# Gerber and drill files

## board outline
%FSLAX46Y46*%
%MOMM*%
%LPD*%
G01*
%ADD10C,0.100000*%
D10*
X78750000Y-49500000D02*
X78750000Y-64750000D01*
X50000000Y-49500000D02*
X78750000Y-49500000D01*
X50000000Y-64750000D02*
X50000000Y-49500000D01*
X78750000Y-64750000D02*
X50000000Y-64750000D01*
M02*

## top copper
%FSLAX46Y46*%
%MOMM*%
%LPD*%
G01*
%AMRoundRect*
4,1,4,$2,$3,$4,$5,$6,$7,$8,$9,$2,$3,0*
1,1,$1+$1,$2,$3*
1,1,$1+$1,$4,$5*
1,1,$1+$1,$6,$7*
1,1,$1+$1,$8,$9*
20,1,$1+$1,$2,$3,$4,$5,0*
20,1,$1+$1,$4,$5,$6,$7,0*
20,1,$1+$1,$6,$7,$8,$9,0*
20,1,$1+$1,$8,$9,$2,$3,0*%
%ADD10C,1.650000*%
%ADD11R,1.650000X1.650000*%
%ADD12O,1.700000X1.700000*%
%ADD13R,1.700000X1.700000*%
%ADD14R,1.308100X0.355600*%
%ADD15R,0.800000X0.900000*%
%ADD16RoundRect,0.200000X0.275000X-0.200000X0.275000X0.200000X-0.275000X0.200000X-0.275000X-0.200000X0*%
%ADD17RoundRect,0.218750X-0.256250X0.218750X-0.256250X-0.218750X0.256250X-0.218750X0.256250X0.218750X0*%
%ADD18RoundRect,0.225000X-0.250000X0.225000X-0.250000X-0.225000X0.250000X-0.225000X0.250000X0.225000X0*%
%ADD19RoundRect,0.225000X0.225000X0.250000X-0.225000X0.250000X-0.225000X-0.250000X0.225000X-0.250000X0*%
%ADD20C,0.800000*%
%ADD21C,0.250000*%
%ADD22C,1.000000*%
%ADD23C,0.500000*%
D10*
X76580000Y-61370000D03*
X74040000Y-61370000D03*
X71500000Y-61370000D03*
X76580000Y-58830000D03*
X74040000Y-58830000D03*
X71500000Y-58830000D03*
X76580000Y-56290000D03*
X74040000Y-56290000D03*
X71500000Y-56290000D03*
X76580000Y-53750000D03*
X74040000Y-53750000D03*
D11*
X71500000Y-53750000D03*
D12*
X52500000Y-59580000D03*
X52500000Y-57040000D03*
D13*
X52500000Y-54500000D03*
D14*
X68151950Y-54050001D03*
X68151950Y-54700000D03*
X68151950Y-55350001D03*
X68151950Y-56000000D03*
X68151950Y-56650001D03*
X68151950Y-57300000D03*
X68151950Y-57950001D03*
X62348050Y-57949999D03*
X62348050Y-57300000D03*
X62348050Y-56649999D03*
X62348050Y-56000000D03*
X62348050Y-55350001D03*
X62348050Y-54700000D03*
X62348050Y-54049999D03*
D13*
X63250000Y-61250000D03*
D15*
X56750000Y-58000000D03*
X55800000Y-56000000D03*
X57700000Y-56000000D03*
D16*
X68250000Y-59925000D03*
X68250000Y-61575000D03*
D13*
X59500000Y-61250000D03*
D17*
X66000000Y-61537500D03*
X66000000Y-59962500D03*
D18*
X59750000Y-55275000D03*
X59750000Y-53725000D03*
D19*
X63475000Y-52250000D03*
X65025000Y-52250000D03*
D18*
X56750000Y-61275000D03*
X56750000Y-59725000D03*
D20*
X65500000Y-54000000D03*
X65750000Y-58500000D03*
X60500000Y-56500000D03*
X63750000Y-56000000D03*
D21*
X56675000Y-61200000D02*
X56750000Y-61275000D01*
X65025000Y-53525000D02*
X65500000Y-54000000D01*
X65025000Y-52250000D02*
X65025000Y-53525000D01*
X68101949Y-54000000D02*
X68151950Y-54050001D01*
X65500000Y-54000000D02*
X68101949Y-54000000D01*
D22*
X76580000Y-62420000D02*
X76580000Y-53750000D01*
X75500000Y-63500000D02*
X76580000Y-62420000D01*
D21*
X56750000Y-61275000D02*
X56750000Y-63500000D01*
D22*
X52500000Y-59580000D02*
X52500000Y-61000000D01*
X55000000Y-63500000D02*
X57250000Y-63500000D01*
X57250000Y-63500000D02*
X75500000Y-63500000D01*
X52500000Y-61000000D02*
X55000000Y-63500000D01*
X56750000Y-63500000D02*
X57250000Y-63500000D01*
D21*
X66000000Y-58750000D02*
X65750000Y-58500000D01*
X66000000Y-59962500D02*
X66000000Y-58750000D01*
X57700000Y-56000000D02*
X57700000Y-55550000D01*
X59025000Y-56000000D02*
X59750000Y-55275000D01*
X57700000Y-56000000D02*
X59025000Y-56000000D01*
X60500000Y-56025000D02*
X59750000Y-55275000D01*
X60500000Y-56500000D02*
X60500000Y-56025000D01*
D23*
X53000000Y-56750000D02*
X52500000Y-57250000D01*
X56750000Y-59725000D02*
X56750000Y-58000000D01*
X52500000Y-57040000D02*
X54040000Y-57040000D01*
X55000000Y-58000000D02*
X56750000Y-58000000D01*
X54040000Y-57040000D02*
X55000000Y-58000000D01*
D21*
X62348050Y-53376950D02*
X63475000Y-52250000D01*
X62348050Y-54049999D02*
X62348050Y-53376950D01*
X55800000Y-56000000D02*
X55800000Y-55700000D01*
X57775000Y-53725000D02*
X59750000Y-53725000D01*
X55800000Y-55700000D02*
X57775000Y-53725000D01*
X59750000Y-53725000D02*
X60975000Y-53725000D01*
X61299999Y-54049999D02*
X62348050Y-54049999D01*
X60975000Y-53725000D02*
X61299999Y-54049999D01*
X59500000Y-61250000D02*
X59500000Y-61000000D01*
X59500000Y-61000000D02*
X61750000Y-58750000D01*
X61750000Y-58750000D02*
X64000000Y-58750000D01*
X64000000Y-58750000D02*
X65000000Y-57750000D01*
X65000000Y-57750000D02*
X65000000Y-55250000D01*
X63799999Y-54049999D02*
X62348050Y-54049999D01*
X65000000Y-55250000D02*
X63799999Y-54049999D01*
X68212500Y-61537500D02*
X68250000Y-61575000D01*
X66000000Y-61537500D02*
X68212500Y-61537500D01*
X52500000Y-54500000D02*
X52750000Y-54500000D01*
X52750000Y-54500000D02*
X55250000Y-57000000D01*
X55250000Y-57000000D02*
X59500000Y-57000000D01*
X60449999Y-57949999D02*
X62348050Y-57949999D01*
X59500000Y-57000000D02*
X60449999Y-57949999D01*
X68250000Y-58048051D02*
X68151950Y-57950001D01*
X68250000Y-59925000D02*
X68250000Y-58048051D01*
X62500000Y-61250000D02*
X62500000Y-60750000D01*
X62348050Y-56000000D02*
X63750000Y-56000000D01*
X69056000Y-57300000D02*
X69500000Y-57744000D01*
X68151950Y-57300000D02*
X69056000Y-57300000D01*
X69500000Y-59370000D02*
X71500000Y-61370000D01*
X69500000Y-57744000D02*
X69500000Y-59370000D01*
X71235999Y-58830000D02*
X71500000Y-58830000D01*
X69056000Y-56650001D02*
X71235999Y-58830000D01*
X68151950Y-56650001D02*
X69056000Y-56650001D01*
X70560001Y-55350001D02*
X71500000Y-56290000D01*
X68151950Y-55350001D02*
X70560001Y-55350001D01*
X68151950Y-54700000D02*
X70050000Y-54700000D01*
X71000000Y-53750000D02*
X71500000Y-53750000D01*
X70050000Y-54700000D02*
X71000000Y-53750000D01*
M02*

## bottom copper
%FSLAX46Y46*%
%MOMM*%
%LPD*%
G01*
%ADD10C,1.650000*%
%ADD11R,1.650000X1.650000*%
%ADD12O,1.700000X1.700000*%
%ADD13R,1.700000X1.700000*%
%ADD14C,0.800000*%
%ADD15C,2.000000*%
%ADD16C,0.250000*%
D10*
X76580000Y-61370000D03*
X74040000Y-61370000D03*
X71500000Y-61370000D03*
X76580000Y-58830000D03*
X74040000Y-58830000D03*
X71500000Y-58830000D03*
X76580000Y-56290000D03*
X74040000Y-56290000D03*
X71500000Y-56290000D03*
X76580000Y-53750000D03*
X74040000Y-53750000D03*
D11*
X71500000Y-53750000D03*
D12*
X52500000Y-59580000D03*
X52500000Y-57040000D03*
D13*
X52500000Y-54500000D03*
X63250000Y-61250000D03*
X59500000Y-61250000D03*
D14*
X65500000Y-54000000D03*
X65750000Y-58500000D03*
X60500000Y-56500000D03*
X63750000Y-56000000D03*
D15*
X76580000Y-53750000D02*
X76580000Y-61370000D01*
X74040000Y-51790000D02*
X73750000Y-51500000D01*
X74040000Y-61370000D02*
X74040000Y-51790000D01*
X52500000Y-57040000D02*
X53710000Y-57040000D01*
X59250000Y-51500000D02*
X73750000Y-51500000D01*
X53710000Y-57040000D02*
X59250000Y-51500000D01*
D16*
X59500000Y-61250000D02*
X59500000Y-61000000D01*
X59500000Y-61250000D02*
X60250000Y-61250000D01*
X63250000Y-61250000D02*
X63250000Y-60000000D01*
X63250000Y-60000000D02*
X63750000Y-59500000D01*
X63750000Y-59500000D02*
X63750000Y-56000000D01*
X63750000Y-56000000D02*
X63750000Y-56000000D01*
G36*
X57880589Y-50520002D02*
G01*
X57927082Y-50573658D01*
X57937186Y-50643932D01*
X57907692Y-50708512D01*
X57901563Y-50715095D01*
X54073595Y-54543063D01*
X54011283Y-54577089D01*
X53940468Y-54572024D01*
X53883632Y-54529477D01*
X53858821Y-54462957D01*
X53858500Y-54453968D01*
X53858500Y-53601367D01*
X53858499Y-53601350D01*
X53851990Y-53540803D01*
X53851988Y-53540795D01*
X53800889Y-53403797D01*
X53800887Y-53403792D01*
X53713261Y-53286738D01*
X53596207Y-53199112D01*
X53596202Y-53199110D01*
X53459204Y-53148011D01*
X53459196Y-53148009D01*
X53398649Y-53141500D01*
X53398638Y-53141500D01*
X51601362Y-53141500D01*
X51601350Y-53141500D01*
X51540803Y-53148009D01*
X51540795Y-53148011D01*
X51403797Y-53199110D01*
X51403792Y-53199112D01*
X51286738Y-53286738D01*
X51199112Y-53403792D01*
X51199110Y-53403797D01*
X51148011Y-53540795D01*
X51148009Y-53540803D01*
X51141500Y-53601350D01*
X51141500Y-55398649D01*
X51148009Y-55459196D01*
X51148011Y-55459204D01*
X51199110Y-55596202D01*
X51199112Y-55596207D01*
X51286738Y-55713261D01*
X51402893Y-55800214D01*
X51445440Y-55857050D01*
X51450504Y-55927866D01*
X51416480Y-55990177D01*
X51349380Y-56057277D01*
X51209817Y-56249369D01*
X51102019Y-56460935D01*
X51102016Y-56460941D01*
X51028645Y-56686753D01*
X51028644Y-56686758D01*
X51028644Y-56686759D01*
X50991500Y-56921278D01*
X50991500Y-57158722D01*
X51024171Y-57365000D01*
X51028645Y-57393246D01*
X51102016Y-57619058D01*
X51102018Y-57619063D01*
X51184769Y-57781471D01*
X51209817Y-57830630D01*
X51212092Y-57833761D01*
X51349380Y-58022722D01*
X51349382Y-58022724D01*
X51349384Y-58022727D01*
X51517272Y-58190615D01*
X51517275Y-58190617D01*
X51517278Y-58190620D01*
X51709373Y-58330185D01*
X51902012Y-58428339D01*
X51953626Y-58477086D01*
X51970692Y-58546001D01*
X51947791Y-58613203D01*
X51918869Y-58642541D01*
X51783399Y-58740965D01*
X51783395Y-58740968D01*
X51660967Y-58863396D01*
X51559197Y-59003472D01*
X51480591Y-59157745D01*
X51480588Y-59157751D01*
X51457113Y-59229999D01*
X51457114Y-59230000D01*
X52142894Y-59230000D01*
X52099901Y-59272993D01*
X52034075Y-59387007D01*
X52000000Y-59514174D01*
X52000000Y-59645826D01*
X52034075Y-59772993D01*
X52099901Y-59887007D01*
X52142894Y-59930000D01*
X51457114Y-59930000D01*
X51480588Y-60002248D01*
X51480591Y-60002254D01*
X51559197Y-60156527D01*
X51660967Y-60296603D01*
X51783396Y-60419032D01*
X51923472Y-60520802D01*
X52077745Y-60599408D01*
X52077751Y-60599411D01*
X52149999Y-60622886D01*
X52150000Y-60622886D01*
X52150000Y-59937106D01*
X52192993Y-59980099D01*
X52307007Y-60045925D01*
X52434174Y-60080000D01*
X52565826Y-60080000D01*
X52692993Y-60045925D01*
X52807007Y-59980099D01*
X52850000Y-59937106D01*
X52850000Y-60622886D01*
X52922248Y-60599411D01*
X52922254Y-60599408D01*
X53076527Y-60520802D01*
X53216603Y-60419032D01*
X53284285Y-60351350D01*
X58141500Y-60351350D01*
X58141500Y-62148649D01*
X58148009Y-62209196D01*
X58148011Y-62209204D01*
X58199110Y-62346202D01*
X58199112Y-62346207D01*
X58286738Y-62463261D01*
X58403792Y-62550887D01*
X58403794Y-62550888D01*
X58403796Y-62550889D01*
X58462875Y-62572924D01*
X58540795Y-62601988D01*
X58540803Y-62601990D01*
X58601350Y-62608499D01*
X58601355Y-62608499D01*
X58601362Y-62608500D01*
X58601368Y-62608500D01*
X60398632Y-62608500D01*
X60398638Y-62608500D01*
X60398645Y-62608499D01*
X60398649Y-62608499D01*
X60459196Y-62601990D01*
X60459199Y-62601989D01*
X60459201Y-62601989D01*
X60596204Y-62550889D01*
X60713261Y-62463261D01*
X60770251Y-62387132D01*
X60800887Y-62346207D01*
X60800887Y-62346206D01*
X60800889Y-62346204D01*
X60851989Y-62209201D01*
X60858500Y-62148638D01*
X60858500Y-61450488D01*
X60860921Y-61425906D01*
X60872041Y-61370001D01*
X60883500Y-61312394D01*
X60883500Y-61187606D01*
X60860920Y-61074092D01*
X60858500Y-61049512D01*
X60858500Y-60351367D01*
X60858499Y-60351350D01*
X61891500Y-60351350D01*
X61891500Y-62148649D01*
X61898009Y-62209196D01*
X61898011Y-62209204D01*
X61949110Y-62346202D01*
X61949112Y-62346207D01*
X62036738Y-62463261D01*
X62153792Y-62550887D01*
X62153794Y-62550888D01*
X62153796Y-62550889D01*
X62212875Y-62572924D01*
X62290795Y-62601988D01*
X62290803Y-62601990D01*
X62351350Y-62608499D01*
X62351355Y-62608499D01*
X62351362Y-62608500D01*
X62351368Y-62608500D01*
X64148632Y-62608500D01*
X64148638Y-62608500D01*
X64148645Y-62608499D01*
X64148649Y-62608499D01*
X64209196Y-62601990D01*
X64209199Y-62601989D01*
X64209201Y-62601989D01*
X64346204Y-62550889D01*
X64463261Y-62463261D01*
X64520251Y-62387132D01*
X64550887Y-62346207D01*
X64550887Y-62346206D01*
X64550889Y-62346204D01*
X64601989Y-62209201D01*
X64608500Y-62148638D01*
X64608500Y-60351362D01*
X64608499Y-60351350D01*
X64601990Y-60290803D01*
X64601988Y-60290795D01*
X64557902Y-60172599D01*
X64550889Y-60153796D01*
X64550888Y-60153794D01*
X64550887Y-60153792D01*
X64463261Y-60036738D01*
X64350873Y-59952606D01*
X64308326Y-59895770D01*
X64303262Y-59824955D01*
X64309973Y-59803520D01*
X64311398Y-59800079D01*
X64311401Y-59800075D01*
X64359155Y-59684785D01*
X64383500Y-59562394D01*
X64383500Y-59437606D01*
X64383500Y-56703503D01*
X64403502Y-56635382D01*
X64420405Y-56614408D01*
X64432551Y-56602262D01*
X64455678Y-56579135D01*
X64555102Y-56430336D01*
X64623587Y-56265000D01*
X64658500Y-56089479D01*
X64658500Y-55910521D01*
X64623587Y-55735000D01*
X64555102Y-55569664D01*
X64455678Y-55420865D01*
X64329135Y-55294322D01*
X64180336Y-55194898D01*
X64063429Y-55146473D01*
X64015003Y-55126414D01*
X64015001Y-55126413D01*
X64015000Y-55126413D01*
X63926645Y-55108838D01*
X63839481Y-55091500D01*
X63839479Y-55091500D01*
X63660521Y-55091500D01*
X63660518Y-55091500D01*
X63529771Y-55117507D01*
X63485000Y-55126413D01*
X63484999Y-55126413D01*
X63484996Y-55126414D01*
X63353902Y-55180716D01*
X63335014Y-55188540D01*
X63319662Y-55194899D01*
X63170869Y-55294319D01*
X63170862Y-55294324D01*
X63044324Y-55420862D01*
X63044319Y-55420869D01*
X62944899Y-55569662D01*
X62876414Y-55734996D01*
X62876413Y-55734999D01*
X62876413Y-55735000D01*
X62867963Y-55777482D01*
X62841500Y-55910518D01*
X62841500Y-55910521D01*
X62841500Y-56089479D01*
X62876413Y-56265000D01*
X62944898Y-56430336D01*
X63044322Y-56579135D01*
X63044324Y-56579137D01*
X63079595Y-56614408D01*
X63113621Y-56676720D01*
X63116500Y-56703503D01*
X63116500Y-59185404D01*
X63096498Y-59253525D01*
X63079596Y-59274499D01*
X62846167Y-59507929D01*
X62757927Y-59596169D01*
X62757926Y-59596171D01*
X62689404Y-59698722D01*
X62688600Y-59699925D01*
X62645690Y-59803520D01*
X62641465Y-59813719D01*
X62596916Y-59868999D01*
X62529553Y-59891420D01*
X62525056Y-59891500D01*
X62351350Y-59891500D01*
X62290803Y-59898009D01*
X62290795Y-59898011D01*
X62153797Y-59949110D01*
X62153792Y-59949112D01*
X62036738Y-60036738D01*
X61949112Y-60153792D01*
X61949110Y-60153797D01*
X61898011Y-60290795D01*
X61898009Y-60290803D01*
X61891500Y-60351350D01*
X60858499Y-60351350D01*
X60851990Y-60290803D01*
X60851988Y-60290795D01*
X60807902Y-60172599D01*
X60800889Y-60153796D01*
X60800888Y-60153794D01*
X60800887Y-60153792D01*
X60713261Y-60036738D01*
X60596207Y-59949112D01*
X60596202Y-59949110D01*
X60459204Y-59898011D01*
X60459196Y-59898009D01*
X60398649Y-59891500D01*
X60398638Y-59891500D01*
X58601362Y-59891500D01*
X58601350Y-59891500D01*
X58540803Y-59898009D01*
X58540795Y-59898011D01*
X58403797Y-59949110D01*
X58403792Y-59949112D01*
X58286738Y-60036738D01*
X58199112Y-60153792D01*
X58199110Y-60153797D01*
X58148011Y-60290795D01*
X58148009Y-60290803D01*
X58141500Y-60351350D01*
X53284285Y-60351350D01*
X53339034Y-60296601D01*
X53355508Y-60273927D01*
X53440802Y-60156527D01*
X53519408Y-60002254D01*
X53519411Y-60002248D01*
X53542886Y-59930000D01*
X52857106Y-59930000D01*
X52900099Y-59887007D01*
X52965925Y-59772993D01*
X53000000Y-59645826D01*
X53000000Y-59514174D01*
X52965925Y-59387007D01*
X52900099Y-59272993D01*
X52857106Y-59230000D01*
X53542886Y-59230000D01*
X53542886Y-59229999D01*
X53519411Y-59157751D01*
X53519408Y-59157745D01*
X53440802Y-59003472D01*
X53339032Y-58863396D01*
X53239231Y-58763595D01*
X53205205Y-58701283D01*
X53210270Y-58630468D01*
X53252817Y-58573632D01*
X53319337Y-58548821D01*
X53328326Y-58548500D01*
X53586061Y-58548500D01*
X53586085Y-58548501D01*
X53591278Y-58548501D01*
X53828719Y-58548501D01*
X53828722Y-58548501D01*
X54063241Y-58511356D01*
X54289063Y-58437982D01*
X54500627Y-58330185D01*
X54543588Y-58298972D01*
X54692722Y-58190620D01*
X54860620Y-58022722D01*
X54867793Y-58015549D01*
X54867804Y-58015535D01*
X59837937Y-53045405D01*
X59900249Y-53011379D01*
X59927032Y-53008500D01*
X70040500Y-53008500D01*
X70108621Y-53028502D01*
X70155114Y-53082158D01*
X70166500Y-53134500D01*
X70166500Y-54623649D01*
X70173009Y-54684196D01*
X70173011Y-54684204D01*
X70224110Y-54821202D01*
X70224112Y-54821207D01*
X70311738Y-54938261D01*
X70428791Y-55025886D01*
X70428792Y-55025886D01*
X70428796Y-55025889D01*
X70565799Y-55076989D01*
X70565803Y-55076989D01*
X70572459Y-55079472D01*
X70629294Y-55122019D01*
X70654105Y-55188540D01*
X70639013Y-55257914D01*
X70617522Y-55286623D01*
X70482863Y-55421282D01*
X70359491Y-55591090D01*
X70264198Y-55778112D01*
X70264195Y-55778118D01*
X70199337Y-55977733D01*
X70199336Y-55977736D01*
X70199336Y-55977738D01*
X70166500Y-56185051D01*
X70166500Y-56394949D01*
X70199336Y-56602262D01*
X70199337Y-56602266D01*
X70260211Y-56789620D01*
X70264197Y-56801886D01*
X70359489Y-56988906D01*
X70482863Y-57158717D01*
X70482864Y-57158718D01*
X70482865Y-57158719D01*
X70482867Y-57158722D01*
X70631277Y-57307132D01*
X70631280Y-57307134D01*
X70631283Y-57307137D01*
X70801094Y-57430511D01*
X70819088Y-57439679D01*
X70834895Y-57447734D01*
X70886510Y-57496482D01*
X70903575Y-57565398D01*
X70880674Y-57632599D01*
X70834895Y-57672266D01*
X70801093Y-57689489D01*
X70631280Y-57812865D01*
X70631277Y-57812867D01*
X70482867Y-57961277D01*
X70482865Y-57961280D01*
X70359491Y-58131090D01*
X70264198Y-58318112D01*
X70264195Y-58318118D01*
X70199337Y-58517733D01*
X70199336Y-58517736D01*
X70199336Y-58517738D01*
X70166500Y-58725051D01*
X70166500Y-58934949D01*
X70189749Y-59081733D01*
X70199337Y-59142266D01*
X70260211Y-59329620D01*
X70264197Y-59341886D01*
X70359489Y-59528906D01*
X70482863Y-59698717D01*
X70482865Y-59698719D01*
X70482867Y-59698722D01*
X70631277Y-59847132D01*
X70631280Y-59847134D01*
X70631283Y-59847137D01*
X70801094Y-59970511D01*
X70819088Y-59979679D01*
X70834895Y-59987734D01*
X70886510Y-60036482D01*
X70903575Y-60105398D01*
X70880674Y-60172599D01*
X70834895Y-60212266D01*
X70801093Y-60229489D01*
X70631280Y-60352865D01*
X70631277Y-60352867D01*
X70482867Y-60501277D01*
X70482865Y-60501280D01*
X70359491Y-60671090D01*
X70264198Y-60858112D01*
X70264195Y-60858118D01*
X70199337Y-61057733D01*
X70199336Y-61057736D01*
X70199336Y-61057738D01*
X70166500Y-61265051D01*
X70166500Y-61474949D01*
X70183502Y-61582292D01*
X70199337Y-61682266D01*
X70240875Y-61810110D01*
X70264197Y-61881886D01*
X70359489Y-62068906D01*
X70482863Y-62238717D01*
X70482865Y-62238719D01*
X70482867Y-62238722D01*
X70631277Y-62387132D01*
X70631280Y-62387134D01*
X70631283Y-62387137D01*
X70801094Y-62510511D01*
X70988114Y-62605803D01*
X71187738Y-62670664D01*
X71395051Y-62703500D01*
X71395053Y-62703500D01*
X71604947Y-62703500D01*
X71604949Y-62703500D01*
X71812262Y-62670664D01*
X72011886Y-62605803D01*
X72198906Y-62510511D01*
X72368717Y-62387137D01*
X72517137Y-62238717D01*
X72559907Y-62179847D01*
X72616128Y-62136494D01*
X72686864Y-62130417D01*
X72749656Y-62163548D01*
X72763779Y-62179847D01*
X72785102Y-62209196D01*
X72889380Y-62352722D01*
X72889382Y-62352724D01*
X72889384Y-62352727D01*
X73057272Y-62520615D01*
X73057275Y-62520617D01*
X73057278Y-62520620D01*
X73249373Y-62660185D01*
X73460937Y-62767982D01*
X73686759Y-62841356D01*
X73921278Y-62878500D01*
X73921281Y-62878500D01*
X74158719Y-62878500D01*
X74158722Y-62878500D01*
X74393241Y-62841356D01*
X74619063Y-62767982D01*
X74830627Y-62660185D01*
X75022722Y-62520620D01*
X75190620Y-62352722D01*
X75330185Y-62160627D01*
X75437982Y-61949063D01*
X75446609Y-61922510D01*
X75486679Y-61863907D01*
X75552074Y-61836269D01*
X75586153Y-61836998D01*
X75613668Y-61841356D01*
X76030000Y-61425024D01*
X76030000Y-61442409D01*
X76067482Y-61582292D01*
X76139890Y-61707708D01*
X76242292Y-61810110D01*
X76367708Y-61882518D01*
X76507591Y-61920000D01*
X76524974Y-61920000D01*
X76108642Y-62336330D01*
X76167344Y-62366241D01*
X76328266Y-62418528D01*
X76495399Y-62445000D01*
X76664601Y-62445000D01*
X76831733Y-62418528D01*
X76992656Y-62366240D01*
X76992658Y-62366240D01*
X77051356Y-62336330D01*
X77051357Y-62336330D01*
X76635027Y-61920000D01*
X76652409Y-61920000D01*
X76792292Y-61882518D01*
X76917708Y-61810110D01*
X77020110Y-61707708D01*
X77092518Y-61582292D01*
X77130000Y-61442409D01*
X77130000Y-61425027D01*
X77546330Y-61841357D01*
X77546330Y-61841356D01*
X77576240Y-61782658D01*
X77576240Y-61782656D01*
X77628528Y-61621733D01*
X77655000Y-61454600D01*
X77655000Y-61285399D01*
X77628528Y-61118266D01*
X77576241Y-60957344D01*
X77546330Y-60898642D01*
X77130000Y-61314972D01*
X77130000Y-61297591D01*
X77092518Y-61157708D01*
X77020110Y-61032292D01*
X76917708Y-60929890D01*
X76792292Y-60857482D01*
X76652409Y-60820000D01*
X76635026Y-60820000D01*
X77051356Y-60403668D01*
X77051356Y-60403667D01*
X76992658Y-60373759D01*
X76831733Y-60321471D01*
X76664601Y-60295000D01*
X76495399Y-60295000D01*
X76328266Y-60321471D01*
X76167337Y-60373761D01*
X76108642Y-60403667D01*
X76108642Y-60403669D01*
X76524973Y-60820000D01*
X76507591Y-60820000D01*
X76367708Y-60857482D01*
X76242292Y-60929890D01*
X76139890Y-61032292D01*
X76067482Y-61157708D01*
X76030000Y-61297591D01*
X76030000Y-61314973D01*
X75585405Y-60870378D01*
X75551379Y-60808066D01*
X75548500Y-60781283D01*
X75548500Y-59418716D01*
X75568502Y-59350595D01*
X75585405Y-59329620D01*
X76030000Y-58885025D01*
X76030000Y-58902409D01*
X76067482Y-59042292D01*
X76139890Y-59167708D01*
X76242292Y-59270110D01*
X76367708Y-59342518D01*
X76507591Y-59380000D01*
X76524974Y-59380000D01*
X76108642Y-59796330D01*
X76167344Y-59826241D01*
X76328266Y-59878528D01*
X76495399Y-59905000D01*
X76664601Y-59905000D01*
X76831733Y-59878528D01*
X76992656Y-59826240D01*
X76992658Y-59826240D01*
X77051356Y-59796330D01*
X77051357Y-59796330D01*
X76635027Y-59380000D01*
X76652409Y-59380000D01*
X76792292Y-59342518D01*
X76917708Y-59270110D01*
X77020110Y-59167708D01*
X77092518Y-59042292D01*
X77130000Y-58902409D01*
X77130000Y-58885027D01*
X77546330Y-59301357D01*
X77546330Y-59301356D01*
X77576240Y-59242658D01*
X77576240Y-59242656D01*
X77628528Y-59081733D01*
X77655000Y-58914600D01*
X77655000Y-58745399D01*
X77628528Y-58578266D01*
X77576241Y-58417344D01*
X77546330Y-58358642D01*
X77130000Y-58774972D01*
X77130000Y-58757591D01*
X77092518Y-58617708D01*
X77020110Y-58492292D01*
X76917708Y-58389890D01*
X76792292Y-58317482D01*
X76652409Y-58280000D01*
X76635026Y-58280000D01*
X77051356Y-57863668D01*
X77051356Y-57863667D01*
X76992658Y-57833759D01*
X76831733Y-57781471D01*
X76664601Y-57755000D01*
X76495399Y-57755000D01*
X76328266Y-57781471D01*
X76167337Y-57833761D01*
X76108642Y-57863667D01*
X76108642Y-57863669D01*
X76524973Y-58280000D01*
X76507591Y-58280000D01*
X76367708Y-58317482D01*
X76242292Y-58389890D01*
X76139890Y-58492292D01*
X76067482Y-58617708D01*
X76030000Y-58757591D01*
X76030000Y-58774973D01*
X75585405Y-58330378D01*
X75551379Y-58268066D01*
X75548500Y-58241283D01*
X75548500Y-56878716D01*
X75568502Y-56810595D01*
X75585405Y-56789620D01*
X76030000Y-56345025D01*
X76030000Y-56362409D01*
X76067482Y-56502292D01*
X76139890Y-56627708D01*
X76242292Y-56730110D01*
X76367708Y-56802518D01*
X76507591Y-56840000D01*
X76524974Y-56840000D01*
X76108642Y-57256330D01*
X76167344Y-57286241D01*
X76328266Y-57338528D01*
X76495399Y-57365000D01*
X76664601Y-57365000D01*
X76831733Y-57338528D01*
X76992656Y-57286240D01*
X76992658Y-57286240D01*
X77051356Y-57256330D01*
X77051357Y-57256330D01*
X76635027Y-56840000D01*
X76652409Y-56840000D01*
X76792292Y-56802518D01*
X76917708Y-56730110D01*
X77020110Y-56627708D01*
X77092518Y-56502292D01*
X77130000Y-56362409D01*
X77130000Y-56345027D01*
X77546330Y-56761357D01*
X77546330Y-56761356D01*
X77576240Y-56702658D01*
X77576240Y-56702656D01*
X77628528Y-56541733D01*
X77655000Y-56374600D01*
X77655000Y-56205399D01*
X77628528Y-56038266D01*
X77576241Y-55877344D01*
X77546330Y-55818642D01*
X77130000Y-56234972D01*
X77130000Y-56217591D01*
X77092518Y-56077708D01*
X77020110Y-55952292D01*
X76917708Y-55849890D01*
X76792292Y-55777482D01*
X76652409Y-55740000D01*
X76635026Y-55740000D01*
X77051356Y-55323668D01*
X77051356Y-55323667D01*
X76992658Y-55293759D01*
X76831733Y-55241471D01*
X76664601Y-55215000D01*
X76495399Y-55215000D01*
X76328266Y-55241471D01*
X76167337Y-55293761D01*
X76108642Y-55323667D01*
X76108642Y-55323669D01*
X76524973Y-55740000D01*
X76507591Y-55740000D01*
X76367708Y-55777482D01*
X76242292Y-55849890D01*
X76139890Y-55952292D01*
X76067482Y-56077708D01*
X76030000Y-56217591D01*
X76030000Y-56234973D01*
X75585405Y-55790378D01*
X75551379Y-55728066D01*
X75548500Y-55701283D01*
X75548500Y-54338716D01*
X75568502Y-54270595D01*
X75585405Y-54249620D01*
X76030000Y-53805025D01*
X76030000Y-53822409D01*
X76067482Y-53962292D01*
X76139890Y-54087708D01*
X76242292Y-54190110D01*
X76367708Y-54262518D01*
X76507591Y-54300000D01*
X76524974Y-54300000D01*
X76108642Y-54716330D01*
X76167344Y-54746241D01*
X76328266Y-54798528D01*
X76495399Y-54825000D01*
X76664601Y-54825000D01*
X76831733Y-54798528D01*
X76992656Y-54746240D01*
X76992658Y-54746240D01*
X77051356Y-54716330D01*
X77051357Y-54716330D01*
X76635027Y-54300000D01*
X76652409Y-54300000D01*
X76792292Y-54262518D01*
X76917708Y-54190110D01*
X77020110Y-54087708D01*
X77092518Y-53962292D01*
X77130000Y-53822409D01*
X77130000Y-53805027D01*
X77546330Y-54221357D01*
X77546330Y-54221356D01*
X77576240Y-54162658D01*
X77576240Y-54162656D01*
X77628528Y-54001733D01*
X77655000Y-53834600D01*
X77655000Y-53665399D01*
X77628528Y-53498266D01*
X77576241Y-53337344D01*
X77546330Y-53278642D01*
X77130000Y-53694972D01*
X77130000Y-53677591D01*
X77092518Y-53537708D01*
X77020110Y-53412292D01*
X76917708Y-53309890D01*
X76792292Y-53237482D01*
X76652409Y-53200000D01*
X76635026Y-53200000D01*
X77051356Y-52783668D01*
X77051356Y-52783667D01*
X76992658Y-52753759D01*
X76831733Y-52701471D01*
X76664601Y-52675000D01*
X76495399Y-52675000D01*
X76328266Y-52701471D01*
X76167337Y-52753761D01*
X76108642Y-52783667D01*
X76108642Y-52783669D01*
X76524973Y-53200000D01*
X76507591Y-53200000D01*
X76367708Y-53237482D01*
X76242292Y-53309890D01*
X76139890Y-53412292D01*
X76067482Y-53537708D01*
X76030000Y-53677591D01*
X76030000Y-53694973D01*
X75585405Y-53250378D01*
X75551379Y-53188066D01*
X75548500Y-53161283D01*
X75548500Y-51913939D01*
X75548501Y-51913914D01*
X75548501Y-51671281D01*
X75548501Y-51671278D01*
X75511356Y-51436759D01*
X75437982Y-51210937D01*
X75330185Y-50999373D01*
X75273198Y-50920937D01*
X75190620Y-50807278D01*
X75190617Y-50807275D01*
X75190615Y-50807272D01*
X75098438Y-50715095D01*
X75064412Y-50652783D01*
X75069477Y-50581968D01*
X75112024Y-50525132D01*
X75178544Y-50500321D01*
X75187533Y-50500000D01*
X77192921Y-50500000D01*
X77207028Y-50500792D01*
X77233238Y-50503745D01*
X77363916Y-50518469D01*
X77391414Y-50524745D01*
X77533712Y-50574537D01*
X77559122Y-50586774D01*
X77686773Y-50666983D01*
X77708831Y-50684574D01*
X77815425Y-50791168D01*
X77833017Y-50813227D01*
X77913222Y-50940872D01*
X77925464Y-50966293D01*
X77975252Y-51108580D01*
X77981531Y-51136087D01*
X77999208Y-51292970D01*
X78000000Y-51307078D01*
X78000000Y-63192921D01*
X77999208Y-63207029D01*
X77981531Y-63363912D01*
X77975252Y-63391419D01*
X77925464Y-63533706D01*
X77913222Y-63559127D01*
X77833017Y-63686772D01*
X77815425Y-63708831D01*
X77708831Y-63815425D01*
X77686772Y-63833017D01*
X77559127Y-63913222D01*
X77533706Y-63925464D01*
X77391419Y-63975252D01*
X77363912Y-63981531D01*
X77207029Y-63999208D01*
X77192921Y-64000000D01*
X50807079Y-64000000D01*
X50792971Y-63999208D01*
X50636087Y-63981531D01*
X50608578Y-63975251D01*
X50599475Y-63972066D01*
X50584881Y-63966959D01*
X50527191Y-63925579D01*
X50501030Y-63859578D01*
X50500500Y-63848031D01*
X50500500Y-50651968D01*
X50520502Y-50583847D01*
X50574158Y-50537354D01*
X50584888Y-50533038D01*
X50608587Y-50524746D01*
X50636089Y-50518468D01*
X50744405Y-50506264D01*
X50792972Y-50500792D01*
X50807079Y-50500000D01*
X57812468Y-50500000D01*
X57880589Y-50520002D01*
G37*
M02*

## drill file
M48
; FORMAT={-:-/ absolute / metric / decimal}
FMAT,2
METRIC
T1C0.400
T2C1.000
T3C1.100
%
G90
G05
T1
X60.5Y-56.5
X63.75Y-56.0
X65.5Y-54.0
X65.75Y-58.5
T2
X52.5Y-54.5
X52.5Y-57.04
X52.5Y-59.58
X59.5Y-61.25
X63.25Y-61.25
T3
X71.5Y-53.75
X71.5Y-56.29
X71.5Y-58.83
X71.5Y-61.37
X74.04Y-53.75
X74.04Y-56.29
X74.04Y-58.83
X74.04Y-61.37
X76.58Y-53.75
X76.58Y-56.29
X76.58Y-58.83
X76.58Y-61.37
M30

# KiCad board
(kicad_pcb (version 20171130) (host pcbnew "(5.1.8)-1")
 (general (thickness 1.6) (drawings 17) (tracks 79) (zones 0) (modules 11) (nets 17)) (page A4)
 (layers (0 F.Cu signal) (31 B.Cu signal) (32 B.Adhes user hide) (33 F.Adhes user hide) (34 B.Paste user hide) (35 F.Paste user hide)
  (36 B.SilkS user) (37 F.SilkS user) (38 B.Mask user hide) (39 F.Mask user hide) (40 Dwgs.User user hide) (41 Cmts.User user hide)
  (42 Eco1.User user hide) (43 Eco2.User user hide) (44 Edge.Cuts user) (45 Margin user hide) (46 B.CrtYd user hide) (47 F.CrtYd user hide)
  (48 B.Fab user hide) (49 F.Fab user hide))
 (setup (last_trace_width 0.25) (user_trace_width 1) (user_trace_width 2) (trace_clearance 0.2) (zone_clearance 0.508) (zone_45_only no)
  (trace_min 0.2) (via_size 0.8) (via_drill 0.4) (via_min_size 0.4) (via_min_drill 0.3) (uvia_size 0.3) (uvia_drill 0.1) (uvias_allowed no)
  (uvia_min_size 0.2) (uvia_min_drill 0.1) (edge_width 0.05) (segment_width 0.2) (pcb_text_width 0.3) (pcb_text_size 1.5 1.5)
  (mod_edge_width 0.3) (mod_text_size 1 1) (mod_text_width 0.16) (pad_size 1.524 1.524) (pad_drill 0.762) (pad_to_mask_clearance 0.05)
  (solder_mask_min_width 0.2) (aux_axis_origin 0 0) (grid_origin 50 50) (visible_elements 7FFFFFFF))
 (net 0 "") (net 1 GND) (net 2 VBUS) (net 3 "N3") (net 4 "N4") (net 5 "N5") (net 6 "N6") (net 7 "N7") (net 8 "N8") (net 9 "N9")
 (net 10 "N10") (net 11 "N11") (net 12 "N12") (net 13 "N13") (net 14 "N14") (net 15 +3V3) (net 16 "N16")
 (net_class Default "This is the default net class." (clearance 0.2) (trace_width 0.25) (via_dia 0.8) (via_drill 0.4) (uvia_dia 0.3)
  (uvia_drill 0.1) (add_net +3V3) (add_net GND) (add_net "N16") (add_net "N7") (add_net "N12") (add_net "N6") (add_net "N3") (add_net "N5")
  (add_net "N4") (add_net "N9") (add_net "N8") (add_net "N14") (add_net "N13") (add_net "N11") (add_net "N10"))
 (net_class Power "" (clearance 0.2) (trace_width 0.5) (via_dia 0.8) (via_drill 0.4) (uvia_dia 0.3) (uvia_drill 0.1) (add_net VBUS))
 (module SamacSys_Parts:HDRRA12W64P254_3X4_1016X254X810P (layer F.Cu) (at 71.5 53.75 270)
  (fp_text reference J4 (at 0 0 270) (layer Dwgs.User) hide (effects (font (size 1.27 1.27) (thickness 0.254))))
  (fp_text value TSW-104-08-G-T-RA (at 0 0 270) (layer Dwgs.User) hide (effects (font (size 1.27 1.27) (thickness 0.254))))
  (pad 12 thru_hole circle (at 7.62 -5.08 270) (size 1.65 1.65) (drill 1.1) (layers *.Cu *.Mask) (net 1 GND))
  (pad 11 thru_hole circle (at 7.62 -2.54 270) (size 1.65 1.65) (drill 1.1) (layers *.Cu *.Mask) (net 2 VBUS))
  (pad 10 thru_hole circle (at 7.62 0 270) (size 1.65 1.65) (drill 1.1) (layers *.Cu *.Mask) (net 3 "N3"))
  (pad 9 thru_hole circle (at 5.08 -5.08 270) (size 1.65 1.65) (drill 1.1) (layers *.Cu *.Mask) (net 1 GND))
  (pad 8 thru_hole circle (at 5.08 -2.54 270) (size 1.65 1.65) (drill 1.1) (layers *.Cu *.Mask) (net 2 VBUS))
  (pad 7 thru_hole circle (at 5.08 0 270) (size 1.65 1.65) (drill 1.1) (layers *.Cu *.Mask) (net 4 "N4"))
  (pad 6 thru_hole circle (at 2.54 -5.08 270) (size 1.65 1.65) (drill 1.1) (layers *.Cu *.Mask) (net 1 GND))
  (pad 5 thru_hole circle (at 2.54 -2.54 270) (size 1.65 1.65) (drill 1.1) (layers *.Cu *.Mask) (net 2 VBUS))
  (pad 4 thru_hole circle (at 2.54 0 270) (size 1.65 1.65) (drill 1.1) (layers *.Cu *.Mask) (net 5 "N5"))
  (pad 3 thru_hole circle (at 0 -5.08 270) (size 1.65 1.65) (drill 1.1) (layers *.Cu *.Mask) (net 1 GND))
  (pad 2 thru_hole circle (at 0 -2.54 270) (size 1.65 1.65) (drill 1.1) (layers *.Cu *.Mask) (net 2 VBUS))
  (pad 1 thru_hole rect (at 0 0 270) (size 1.65 1.65) (drill 1.1) (layers *.Cu *.Mask) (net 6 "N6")))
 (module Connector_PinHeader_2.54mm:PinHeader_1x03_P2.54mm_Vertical (layer F.Cu) (at 52.5 54.5)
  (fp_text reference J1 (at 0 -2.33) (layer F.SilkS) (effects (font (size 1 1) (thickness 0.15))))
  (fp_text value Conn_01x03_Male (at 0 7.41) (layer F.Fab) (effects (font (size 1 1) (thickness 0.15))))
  (pad 3 thru_hole oval (at 0 5.08) (size 1.7 1.7) (drill 1) (layers *.Cu *.Mask) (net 1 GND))
  (pad 2 thru_hole oval (at 0 2.54) (size 1.7 1.7) (drill 1) (layers *.Cu *.Mask) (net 2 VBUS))
  (pad 1 thru_hole rect (at 0 0) (size 1.7 1.7) (drill 1) (layers *.Cu *.Mask) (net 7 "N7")))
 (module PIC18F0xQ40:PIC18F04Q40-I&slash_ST (layer F.Cu) (at 65.25 56)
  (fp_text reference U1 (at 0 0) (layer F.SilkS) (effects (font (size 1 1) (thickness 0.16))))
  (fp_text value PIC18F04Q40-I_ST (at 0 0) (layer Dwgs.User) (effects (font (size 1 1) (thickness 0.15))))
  (pad 14 smd rect (at 2.90195 -1.949999) (size 1.3081 0.3556) (layers F.Cu F.Paste F.Mask) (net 1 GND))
  (pad 13 smd rect (at 2.90195 -1.3) (size 1.3081 0.3556) (layers F.Cu F.Paste F.Mask) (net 6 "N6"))
  (pad 12 smd rect (at 2.90195 -0.649999) (size 1.3081 0.3556) (layers F.Cu F.Paste F.Mask) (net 5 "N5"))
  (pad 11 smd rect (at 2.90195 0) (size 1.3081 0.3556) (layers F.Cu F.Paste F.Mask) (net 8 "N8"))
  (pad 10 smd rect (at 2.90195 0.650001) (size 1.3081 0.3556) (layers F.Cu F.Paste F.Mask) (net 4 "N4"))
  (pad 9 smd rect (at 2.90195 1.3) (size 1.3081 0.3556) (layers F.Cu F.Paste F.Mask) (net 3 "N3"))
  (pad 8 smd rect (at 2.90195 1.950001) (size 1.3081 0.3556) (layers F.Cu F.Paste F.Mask) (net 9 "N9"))
  (pad 7 smd rect (at -2.90195 1.949999) (size 1.3081 0.3556) (layers F.Cu F.Paste F.Mask) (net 7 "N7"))
  (pad 6 smd rect (at -2.90195 1.3) (size 1.3081 0.3556) (layers F.Cu F.Paste F.Mask) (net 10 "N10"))
  (pad 5 smd rect (at -2.90195 0.649999) (size 1.3081 0.3556) (layers F.Cu F.Paste F.Mask) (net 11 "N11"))
  (pad 4 smd rect (at -2.90195 0) (size 1.3081 0.3556) (layers F.Cu F.Paste F.Mask) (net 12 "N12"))
  (pad 3 smd rect (at -2.90195 -0.649999) (size 1.3081 0.3556) (layers F.Cu F.Paste F.Mask) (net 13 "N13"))
  (pad 2 smd rect (at -2.90195 -1.3) (size 1.3081 0.3556) (layers F.Cu F.Paste F.Mask) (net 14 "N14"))
  (pad 1 smd rect (at -2.90195 -1.950001) (size 1.3081 0.3556) (layers F.Cu F.Paste F.Mask) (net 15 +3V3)))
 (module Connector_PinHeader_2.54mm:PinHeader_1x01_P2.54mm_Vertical (layer F.Cu) (at 63.25 61.25)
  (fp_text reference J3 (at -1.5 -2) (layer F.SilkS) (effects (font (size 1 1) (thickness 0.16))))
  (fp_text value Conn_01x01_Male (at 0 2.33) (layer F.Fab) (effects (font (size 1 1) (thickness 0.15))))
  (pad 1 thru_hole rect (at 0 0) (size 1.7 1.7) (drill 1) (layers *.Cu *.Mask) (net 12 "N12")))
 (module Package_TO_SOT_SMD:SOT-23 (layer F.Cu) (at 56.75 57 270)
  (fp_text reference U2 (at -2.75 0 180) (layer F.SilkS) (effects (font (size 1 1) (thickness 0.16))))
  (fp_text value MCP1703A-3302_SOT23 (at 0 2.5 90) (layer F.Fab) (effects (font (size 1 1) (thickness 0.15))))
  (pad 3 smd rect (at 1 0 270) (size 0.9 0.8) (layers F.Cu F.Paste F.Mask) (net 2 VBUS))
  (pad 2 smd rect (at -1 0.95 270) (size 0.9 0.8) (layers F.Cu F.Paste F.Mask) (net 15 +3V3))
  (pad 1 smd rect (at -1 -0.95 270) (size 0.9 0.8) (layers F.Cu F.Paste F.Mask) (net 1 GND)))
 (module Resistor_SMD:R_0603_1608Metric (layer F.Cu) (at 68.25 60.75 90)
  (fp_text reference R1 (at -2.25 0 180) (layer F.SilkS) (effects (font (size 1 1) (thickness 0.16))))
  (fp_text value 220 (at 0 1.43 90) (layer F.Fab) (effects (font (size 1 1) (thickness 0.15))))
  (pad 2 smd roundrect (at 0.825 0 90) (size 0.8 0.95) (layers F.Cu F.Paste F.Mask) (roundrect_rratio 0.25) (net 9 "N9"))
  (pad 1 smd roundrect (at -0.825 0 90) (size 0.8 0.95) (layers F.Cu F.Paste F.Mask) (roundrect_rratio 0.25) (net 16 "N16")))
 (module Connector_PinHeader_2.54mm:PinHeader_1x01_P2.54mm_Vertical (layer F.Cu) (at 59.5 61.25)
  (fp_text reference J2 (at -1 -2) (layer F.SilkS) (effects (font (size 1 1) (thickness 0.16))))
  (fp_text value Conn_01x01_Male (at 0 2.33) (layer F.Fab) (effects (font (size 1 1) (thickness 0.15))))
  (pad 1 thru_hole rect (at 0 0) (size 1.7 1.7) (drill 1) (layers *.Cu *.Mask) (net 15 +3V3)))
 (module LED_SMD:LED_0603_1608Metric (layer F.Cu) (at 66 60.75 270)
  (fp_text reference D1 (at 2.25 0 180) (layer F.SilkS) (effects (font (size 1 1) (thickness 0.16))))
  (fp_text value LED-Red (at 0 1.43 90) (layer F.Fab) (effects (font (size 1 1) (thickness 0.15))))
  (pad 2 smd roundrect (at 0.7875 0 270) (size 0.875 0.95) (layers F.Cu F.Paste F.Mask) (roundrect_rratio 0.25) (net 16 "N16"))
  (pad 1 smd roundrect (at -0.7875 0 270) (size 0.875 0.95) (layers F.Cu F.Paste F.Mask) (roundrect_rratio 0.25) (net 1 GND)))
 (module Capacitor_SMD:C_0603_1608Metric (layer F.Cu) (at 59.75 54.5 270)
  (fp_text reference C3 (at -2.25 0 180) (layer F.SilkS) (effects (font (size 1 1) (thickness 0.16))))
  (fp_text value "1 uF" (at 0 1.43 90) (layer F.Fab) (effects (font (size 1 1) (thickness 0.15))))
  (pad 2 smd roundrect (at 0.775 0 270) (size 0.9 0.95) (layers F.Cu F.Paste F.Mask) (roundrect_rratio 0.25) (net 1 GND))
  (pad 1 smd roundrect (at -0.775 0 270) (size 0.9 0.95) (layers F.Cu F.Paste F.Mask) (roundrect_rratio 0.25) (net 15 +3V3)))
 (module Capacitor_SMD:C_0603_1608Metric (layer F.Cu) (at 64.25 52.25 180)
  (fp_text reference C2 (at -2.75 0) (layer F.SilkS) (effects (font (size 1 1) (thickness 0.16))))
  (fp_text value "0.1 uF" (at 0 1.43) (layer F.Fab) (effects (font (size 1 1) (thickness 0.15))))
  (pad 2 smd roundrect (at 0.775 0 180) (size 0.9 0.95) (layers F.Cu F.Paste F.Mask) (roundrect_rratio 0.25) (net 15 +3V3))
  (pad 1 smd roundrect (at -0.775 0 180) (size 0.9 0.95) (layers F.Cu F.Paste F.Mask) (roundrect_rratio 0.25) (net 1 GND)))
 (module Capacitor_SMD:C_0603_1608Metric (layer F.Cu) (at 56.75 60.5 270)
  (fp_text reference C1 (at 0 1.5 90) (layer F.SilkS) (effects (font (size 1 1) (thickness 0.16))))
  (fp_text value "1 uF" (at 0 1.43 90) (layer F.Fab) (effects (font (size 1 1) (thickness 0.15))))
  (pad 2 smd roundrect (at 0.775 0 270) (size 0.9 0.95) (layers F.Cu F.Paste F.Mask) (roundrect_rratio 0.25) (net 1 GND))
  (pad 1 smd roundrect (at -0.775 0 270) (size 0.9 0.95) (layers F.Cu F.Paste F.Mask) (roundrect_rratio 0.25) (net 2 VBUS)))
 (gr_line (start 78.75 49.5) (end 78.75 64.75) (layer Edge.Cuts) (width 0.1))
 (gr_line (start 50 49.5) (end 78.75 49.5) (layer Edge.Cuts) (width 0.1))
 (gr_line (start 50 64.75) (end 50 49.5) (layer Edge.Cuts) (width 0.1))
 (gr_line (start 78.75 64.75) (end 50 64.75) (layer Edge.Cuts) (width 0.1))
 (segment (start 56.675 61.2) (end 56.75 61.275) (width 0.25) (layer F.Cu) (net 1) (status 30))
 (via (at 65.5 54) (size 0.8) (drill 0.4) (layers F.Cu B.Cu) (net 1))
 (segment (start 65.025 53.525) (end 65.5 54) (width 0.25) (layer F.Cu) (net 1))
 (segment (start 65.025 52.25) (end 65.025 53.525) (width 0.25) (layer F.Cu) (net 1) (status 10))
 (segment (start 68.101949 54) (end 68.15195 54.050001) (width 0.25) (layer F.Cu) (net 1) (status 30))
 (segment (start 65.5 54) (end 68.101949 54) (width 0.25) (layer F.Cu) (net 1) (status 20))
 (segment (start 76.58 53.75) (end 76.58 61.37) (width 2) (layer B.Cu) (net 1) (status 30))
 (segment (start 76.58 62.42) (end 76.58 53.75) (width 1) (layer F.Cu) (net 1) (status 20))
 (segment (start 75.5 63.5) (end 76.58 62.42) (width 1) (layer F.Cu) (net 1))
 (segment (start 56.75 61.275) (end 56.75 63.5) (width 0.25) (layer F.Cu) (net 1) (status 10))
 (segment (start 52.5 59.58) (end 52.5 61) (width 1) (layer F.Cu) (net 1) (status 10))
 (segment (start 55 63.5) (end 57.25 63.5) (width 1) (layer F.Cu) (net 1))
 (segment (start 57.25 63.5) (end 75.5 63.5) (width 1) (layer F.Cu) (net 1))
 (segment (start 52.5 61) (end 55 63.5) (width 1) (layer F.Cu) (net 1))
 (segment (start 56.75 63.5) (end 57.25 63.5) (width 1) (layer F.Cu) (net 1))
 (via (at 65.75 58.5) (size 0.8) (drill 0.4) (layers F.Cu B.Cu) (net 1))
 (segment (start 66 58.75) (end 65.75 58.5) (width 0.25) (layer F.Cu) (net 1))
 (segment (start 66 59.9625) (end 66 58.75) (width 0.25) (layer F.Cu) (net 1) (status 10))
 (segment (start 57.7 56) (end 57.7 55.55) (width 0.25) (layer F.Cu) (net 1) (status 30))
 (segment (start 59.025 56) (end 59.75 55.275) (width 0.25) (layer F.Cu) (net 1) (status 20))
 (segment (start 57.7 56) (end 59.025 56) (width 0.25) (layer F.Cu) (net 1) (status 10))
 (via (at 60.5 56.5) (size 0.8) (drill 0.4) (layers F.Cu B.Cu) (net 1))
 (segment (start 60.5 56.025) (end 59.75 55.275) (width 0.25) (layer F.Cu) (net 1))
 (segment (start 60.5 56.5) (end 60.5 56.025) (width 0.25) (layer F.Cu) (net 1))
 (segment (start 74.04 51.79) (end 73.75 51.5) (width 2) (layer B.Cu) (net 2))
 (segment (start 74.04 61.37) (end 74.04 51.79) (width 2) (layer B.Cu) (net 2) (status 10))
 (segment (start 53 56.75) (end 52.5 57.25) (width 0.5) (layer F.Cu) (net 2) (status 30))
 (segment (start 52.5 57.04) (end 53.71 57.04) (width 2) (layer B.Cu) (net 2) (status 10))
 (segment (start 59.25 51.5) (end 73.75 51.5) (width 2) (layer B.Cu) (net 2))
 (segment (start 53.71 57.04) (end 59.25 51.5) (width 2) (layer B.Cu) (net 2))
 (segment (start 56.75 59.725) (end 56.75 58) (width 0.5) (layer F.Cu) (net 2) (status 30))
 (segment (start 52.5 57.04) (end 54.04 57.04) (width 0.5) (layer F.Cu) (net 2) (status 10))
 (segment (start 55 58) (end 56.75 58) (width 0.5) (layer F.Cu) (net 2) (status 20))
 (segment (start 54.04 57.04) (end 55 58) (width 0.5) (layer F.Cu) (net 2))
 (segment (start 62.34805 53.37695) (end 63.475 52.25) (width 0.25) (layer F.Cu) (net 15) (status 20))
 (segment (start 62.34805 54.049999) (end 62.34805 53.37695) (width 0.25) (layer F.Cu) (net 15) (status 10))
 (segment (start 59.5 61.25) (end 59.5 61) (width 0.25) (layer B.Cu) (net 15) (status 30))
 (segment (start 55.8 56) (end 55.8 55.7) (width 0.25) (layer F.Cu) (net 15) (status 30))
 (segment (start 57.775 53.725) (end 59.75 53.725) (width 0.25) (layer F.Cu) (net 15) (status 20))
 (segment (start 55.8 55.7) (end 57.775 53.725) (width 0.25) (layer F.Cu) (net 15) (status 10))
 (segment (start 59.75 53.725) (end 60.975 53.725) (width 0.25) (layer F.Cu) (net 15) (status 10))
 (segment (start 61.299999 54.049999) (end 62.34805 54.049999) (width 0.25) (layer F.Cu) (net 15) (status 20))
 (segment (start 60.975 53.725) (end 61.299999 54.049999) (width 0.25) (layer F.Cu) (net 15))
 (segment (start 59.5 61.25) (end 60.25 61.25) (width 0.25) (layer B.Cu) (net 15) (status 30))
 (segment (start 59.5 61.25) (end 59.5 61) (width 0.25) (layer F.Cu) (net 15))
 (segment (start 59.5 61) (end 61.75 58.75) (width 0.25) (layer F.Cu) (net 15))
 (segment (start 61.75 58.75) (end 64 58.75) (width 0.25) (layer F.Cu) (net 15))
 (segment (start 64 58.75) (end 65 57.75) (width 0.25) (layer F.Cu) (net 15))
 (segment (start 65 57.75) (end 65 55.25) (width 0.25) (layer F.Cu) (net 15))
 (segment (start 63.799999 54.049999) (end 62.34805 54.049999) (width 0.25) (layer F.Cu) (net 15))
 (segment (start 65 55.25) (end 63.799999 54.049999) (width 0.25) (layer F.Cu) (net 15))
 (segment (start 68.2125 61.5375) (end 68.25 61.575) (width 0.25) (layer F.Cu) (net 16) (status 30))
 (segment (start 66 61.5375) (end 68.2125 61.5375) (width 0.25) (layer F.Cu) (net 16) (status 30))
 (segment (start 52.5 54.5) (end 52.75 54.5) (width 0.25) (layer F.Cu) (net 7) (status 30))
 (segment (start 52.75 54.5) (end 55.25 57) (width 0.25) (layer F.Cu) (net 7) (status 10))
 (segment (start 55.25 57) (end 59.5 57) (width 0.25) (layer F.Cu) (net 7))
 (segment (start 60.449999 57.949999) (end 62.34805 57.949999) (width 0.25) (layer F.Cu) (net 7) (status 20))
 (segment (start 59.5 57) (end 60.449999 57.949999) (width 0.25) (layer F.Cu) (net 7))
 (segment (start 68.25 58.048051) (end 68.15195 57.950001) (width 0.25) (layer F.Cu) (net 9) (status 30))
 (segment (start 68.25 59.925) (end 68.25 58.048051) (width 0.25) (layer F.Cu) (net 9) (status 30))
 (segment (start 62.5 61.25) (end 62.5 60.75) (width 0.25) (layer F.Cu) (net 12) (status 30))
 (segment (start 63.25 61.25) (end 63.25 60) (width 0.25) (layer B.Cu) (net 12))
 (segment (start 63.25 60) (end 63.75 59.5) (width 0.25) (layer B.Cu) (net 12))
 (segment (start 63.75 59.5) (end 63.75 56) (width 0.25) (layer B.Cu) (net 12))
 (segment (start 63.75 56) (end 63.75 56) (width 0.25) (layer B.Cu) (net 12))
 (via (at 63.75 56) (size 0.8) (drill 0.4) (layers F.Cu B.Cu) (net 12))
 (segment (start 62.34805 56) (end 63.75 56) (width 0.25) (layer F.Cu) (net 12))
 (segment (start 69.056 57.3) (end 69.5 57.744) (width 0.25) (layer F.Cu) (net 3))
 (segment (start 68.15195 57.3) (end 69.056 57.3) (width 0.25) (layer F.Cu) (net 3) (status 10))
 (segment (start 69.5 59.37) (end 71.5 61.37) (width 0.25) (layer F.Cu) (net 3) (status 20))
 (segment (start 69.5 57.744) (end 69.5 59.37) (width 0.25) (layer F.Cu) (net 3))
 (segment (start 71.235999 58.83) (end 71.5 58.83) (width 0.25) (layer F.Cu) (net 4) (status 30))
 (segment (start 69.056 56.650001) (end 71.235999 58.83) (width 0.25) (layer F.Cu) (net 4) (status 20))
 (segment (start 68.15195 56.650001) (end 69.056 56.650001) (width 0.25) (layer F.Cu) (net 4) (status 10))
 (segment (start 70.560001 55.350001) (end 71.5 56.29) (width 0.25) (layer F.Cu) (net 5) (status 20))
 (segment (start 68.15195 55.350001) (end 70.560001 55.350001) (width 0.25) (layer F.Cu) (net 5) (status 10))
 (segment (start 68.15195 54.7) (end 70.05 54.7) (width 0.25) (layer F.Cu) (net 6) (status 10))
 (segment (start 71 53.75) (end 71.5 53.75) (width 0.25) (layer F.Cu) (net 6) (status 30))
 (segment (start 70.05 54.7) (end 71 53.75) (width 0.25) (layer F.Cu) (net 6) (status 20))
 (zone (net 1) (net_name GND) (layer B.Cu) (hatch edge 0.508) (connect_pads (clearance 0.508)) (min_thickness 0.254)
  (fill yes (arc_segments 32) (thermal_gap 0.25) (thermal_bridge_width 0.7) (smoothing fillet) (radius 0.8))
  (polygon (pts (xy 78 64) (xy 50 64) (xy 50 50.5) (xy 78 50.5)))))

